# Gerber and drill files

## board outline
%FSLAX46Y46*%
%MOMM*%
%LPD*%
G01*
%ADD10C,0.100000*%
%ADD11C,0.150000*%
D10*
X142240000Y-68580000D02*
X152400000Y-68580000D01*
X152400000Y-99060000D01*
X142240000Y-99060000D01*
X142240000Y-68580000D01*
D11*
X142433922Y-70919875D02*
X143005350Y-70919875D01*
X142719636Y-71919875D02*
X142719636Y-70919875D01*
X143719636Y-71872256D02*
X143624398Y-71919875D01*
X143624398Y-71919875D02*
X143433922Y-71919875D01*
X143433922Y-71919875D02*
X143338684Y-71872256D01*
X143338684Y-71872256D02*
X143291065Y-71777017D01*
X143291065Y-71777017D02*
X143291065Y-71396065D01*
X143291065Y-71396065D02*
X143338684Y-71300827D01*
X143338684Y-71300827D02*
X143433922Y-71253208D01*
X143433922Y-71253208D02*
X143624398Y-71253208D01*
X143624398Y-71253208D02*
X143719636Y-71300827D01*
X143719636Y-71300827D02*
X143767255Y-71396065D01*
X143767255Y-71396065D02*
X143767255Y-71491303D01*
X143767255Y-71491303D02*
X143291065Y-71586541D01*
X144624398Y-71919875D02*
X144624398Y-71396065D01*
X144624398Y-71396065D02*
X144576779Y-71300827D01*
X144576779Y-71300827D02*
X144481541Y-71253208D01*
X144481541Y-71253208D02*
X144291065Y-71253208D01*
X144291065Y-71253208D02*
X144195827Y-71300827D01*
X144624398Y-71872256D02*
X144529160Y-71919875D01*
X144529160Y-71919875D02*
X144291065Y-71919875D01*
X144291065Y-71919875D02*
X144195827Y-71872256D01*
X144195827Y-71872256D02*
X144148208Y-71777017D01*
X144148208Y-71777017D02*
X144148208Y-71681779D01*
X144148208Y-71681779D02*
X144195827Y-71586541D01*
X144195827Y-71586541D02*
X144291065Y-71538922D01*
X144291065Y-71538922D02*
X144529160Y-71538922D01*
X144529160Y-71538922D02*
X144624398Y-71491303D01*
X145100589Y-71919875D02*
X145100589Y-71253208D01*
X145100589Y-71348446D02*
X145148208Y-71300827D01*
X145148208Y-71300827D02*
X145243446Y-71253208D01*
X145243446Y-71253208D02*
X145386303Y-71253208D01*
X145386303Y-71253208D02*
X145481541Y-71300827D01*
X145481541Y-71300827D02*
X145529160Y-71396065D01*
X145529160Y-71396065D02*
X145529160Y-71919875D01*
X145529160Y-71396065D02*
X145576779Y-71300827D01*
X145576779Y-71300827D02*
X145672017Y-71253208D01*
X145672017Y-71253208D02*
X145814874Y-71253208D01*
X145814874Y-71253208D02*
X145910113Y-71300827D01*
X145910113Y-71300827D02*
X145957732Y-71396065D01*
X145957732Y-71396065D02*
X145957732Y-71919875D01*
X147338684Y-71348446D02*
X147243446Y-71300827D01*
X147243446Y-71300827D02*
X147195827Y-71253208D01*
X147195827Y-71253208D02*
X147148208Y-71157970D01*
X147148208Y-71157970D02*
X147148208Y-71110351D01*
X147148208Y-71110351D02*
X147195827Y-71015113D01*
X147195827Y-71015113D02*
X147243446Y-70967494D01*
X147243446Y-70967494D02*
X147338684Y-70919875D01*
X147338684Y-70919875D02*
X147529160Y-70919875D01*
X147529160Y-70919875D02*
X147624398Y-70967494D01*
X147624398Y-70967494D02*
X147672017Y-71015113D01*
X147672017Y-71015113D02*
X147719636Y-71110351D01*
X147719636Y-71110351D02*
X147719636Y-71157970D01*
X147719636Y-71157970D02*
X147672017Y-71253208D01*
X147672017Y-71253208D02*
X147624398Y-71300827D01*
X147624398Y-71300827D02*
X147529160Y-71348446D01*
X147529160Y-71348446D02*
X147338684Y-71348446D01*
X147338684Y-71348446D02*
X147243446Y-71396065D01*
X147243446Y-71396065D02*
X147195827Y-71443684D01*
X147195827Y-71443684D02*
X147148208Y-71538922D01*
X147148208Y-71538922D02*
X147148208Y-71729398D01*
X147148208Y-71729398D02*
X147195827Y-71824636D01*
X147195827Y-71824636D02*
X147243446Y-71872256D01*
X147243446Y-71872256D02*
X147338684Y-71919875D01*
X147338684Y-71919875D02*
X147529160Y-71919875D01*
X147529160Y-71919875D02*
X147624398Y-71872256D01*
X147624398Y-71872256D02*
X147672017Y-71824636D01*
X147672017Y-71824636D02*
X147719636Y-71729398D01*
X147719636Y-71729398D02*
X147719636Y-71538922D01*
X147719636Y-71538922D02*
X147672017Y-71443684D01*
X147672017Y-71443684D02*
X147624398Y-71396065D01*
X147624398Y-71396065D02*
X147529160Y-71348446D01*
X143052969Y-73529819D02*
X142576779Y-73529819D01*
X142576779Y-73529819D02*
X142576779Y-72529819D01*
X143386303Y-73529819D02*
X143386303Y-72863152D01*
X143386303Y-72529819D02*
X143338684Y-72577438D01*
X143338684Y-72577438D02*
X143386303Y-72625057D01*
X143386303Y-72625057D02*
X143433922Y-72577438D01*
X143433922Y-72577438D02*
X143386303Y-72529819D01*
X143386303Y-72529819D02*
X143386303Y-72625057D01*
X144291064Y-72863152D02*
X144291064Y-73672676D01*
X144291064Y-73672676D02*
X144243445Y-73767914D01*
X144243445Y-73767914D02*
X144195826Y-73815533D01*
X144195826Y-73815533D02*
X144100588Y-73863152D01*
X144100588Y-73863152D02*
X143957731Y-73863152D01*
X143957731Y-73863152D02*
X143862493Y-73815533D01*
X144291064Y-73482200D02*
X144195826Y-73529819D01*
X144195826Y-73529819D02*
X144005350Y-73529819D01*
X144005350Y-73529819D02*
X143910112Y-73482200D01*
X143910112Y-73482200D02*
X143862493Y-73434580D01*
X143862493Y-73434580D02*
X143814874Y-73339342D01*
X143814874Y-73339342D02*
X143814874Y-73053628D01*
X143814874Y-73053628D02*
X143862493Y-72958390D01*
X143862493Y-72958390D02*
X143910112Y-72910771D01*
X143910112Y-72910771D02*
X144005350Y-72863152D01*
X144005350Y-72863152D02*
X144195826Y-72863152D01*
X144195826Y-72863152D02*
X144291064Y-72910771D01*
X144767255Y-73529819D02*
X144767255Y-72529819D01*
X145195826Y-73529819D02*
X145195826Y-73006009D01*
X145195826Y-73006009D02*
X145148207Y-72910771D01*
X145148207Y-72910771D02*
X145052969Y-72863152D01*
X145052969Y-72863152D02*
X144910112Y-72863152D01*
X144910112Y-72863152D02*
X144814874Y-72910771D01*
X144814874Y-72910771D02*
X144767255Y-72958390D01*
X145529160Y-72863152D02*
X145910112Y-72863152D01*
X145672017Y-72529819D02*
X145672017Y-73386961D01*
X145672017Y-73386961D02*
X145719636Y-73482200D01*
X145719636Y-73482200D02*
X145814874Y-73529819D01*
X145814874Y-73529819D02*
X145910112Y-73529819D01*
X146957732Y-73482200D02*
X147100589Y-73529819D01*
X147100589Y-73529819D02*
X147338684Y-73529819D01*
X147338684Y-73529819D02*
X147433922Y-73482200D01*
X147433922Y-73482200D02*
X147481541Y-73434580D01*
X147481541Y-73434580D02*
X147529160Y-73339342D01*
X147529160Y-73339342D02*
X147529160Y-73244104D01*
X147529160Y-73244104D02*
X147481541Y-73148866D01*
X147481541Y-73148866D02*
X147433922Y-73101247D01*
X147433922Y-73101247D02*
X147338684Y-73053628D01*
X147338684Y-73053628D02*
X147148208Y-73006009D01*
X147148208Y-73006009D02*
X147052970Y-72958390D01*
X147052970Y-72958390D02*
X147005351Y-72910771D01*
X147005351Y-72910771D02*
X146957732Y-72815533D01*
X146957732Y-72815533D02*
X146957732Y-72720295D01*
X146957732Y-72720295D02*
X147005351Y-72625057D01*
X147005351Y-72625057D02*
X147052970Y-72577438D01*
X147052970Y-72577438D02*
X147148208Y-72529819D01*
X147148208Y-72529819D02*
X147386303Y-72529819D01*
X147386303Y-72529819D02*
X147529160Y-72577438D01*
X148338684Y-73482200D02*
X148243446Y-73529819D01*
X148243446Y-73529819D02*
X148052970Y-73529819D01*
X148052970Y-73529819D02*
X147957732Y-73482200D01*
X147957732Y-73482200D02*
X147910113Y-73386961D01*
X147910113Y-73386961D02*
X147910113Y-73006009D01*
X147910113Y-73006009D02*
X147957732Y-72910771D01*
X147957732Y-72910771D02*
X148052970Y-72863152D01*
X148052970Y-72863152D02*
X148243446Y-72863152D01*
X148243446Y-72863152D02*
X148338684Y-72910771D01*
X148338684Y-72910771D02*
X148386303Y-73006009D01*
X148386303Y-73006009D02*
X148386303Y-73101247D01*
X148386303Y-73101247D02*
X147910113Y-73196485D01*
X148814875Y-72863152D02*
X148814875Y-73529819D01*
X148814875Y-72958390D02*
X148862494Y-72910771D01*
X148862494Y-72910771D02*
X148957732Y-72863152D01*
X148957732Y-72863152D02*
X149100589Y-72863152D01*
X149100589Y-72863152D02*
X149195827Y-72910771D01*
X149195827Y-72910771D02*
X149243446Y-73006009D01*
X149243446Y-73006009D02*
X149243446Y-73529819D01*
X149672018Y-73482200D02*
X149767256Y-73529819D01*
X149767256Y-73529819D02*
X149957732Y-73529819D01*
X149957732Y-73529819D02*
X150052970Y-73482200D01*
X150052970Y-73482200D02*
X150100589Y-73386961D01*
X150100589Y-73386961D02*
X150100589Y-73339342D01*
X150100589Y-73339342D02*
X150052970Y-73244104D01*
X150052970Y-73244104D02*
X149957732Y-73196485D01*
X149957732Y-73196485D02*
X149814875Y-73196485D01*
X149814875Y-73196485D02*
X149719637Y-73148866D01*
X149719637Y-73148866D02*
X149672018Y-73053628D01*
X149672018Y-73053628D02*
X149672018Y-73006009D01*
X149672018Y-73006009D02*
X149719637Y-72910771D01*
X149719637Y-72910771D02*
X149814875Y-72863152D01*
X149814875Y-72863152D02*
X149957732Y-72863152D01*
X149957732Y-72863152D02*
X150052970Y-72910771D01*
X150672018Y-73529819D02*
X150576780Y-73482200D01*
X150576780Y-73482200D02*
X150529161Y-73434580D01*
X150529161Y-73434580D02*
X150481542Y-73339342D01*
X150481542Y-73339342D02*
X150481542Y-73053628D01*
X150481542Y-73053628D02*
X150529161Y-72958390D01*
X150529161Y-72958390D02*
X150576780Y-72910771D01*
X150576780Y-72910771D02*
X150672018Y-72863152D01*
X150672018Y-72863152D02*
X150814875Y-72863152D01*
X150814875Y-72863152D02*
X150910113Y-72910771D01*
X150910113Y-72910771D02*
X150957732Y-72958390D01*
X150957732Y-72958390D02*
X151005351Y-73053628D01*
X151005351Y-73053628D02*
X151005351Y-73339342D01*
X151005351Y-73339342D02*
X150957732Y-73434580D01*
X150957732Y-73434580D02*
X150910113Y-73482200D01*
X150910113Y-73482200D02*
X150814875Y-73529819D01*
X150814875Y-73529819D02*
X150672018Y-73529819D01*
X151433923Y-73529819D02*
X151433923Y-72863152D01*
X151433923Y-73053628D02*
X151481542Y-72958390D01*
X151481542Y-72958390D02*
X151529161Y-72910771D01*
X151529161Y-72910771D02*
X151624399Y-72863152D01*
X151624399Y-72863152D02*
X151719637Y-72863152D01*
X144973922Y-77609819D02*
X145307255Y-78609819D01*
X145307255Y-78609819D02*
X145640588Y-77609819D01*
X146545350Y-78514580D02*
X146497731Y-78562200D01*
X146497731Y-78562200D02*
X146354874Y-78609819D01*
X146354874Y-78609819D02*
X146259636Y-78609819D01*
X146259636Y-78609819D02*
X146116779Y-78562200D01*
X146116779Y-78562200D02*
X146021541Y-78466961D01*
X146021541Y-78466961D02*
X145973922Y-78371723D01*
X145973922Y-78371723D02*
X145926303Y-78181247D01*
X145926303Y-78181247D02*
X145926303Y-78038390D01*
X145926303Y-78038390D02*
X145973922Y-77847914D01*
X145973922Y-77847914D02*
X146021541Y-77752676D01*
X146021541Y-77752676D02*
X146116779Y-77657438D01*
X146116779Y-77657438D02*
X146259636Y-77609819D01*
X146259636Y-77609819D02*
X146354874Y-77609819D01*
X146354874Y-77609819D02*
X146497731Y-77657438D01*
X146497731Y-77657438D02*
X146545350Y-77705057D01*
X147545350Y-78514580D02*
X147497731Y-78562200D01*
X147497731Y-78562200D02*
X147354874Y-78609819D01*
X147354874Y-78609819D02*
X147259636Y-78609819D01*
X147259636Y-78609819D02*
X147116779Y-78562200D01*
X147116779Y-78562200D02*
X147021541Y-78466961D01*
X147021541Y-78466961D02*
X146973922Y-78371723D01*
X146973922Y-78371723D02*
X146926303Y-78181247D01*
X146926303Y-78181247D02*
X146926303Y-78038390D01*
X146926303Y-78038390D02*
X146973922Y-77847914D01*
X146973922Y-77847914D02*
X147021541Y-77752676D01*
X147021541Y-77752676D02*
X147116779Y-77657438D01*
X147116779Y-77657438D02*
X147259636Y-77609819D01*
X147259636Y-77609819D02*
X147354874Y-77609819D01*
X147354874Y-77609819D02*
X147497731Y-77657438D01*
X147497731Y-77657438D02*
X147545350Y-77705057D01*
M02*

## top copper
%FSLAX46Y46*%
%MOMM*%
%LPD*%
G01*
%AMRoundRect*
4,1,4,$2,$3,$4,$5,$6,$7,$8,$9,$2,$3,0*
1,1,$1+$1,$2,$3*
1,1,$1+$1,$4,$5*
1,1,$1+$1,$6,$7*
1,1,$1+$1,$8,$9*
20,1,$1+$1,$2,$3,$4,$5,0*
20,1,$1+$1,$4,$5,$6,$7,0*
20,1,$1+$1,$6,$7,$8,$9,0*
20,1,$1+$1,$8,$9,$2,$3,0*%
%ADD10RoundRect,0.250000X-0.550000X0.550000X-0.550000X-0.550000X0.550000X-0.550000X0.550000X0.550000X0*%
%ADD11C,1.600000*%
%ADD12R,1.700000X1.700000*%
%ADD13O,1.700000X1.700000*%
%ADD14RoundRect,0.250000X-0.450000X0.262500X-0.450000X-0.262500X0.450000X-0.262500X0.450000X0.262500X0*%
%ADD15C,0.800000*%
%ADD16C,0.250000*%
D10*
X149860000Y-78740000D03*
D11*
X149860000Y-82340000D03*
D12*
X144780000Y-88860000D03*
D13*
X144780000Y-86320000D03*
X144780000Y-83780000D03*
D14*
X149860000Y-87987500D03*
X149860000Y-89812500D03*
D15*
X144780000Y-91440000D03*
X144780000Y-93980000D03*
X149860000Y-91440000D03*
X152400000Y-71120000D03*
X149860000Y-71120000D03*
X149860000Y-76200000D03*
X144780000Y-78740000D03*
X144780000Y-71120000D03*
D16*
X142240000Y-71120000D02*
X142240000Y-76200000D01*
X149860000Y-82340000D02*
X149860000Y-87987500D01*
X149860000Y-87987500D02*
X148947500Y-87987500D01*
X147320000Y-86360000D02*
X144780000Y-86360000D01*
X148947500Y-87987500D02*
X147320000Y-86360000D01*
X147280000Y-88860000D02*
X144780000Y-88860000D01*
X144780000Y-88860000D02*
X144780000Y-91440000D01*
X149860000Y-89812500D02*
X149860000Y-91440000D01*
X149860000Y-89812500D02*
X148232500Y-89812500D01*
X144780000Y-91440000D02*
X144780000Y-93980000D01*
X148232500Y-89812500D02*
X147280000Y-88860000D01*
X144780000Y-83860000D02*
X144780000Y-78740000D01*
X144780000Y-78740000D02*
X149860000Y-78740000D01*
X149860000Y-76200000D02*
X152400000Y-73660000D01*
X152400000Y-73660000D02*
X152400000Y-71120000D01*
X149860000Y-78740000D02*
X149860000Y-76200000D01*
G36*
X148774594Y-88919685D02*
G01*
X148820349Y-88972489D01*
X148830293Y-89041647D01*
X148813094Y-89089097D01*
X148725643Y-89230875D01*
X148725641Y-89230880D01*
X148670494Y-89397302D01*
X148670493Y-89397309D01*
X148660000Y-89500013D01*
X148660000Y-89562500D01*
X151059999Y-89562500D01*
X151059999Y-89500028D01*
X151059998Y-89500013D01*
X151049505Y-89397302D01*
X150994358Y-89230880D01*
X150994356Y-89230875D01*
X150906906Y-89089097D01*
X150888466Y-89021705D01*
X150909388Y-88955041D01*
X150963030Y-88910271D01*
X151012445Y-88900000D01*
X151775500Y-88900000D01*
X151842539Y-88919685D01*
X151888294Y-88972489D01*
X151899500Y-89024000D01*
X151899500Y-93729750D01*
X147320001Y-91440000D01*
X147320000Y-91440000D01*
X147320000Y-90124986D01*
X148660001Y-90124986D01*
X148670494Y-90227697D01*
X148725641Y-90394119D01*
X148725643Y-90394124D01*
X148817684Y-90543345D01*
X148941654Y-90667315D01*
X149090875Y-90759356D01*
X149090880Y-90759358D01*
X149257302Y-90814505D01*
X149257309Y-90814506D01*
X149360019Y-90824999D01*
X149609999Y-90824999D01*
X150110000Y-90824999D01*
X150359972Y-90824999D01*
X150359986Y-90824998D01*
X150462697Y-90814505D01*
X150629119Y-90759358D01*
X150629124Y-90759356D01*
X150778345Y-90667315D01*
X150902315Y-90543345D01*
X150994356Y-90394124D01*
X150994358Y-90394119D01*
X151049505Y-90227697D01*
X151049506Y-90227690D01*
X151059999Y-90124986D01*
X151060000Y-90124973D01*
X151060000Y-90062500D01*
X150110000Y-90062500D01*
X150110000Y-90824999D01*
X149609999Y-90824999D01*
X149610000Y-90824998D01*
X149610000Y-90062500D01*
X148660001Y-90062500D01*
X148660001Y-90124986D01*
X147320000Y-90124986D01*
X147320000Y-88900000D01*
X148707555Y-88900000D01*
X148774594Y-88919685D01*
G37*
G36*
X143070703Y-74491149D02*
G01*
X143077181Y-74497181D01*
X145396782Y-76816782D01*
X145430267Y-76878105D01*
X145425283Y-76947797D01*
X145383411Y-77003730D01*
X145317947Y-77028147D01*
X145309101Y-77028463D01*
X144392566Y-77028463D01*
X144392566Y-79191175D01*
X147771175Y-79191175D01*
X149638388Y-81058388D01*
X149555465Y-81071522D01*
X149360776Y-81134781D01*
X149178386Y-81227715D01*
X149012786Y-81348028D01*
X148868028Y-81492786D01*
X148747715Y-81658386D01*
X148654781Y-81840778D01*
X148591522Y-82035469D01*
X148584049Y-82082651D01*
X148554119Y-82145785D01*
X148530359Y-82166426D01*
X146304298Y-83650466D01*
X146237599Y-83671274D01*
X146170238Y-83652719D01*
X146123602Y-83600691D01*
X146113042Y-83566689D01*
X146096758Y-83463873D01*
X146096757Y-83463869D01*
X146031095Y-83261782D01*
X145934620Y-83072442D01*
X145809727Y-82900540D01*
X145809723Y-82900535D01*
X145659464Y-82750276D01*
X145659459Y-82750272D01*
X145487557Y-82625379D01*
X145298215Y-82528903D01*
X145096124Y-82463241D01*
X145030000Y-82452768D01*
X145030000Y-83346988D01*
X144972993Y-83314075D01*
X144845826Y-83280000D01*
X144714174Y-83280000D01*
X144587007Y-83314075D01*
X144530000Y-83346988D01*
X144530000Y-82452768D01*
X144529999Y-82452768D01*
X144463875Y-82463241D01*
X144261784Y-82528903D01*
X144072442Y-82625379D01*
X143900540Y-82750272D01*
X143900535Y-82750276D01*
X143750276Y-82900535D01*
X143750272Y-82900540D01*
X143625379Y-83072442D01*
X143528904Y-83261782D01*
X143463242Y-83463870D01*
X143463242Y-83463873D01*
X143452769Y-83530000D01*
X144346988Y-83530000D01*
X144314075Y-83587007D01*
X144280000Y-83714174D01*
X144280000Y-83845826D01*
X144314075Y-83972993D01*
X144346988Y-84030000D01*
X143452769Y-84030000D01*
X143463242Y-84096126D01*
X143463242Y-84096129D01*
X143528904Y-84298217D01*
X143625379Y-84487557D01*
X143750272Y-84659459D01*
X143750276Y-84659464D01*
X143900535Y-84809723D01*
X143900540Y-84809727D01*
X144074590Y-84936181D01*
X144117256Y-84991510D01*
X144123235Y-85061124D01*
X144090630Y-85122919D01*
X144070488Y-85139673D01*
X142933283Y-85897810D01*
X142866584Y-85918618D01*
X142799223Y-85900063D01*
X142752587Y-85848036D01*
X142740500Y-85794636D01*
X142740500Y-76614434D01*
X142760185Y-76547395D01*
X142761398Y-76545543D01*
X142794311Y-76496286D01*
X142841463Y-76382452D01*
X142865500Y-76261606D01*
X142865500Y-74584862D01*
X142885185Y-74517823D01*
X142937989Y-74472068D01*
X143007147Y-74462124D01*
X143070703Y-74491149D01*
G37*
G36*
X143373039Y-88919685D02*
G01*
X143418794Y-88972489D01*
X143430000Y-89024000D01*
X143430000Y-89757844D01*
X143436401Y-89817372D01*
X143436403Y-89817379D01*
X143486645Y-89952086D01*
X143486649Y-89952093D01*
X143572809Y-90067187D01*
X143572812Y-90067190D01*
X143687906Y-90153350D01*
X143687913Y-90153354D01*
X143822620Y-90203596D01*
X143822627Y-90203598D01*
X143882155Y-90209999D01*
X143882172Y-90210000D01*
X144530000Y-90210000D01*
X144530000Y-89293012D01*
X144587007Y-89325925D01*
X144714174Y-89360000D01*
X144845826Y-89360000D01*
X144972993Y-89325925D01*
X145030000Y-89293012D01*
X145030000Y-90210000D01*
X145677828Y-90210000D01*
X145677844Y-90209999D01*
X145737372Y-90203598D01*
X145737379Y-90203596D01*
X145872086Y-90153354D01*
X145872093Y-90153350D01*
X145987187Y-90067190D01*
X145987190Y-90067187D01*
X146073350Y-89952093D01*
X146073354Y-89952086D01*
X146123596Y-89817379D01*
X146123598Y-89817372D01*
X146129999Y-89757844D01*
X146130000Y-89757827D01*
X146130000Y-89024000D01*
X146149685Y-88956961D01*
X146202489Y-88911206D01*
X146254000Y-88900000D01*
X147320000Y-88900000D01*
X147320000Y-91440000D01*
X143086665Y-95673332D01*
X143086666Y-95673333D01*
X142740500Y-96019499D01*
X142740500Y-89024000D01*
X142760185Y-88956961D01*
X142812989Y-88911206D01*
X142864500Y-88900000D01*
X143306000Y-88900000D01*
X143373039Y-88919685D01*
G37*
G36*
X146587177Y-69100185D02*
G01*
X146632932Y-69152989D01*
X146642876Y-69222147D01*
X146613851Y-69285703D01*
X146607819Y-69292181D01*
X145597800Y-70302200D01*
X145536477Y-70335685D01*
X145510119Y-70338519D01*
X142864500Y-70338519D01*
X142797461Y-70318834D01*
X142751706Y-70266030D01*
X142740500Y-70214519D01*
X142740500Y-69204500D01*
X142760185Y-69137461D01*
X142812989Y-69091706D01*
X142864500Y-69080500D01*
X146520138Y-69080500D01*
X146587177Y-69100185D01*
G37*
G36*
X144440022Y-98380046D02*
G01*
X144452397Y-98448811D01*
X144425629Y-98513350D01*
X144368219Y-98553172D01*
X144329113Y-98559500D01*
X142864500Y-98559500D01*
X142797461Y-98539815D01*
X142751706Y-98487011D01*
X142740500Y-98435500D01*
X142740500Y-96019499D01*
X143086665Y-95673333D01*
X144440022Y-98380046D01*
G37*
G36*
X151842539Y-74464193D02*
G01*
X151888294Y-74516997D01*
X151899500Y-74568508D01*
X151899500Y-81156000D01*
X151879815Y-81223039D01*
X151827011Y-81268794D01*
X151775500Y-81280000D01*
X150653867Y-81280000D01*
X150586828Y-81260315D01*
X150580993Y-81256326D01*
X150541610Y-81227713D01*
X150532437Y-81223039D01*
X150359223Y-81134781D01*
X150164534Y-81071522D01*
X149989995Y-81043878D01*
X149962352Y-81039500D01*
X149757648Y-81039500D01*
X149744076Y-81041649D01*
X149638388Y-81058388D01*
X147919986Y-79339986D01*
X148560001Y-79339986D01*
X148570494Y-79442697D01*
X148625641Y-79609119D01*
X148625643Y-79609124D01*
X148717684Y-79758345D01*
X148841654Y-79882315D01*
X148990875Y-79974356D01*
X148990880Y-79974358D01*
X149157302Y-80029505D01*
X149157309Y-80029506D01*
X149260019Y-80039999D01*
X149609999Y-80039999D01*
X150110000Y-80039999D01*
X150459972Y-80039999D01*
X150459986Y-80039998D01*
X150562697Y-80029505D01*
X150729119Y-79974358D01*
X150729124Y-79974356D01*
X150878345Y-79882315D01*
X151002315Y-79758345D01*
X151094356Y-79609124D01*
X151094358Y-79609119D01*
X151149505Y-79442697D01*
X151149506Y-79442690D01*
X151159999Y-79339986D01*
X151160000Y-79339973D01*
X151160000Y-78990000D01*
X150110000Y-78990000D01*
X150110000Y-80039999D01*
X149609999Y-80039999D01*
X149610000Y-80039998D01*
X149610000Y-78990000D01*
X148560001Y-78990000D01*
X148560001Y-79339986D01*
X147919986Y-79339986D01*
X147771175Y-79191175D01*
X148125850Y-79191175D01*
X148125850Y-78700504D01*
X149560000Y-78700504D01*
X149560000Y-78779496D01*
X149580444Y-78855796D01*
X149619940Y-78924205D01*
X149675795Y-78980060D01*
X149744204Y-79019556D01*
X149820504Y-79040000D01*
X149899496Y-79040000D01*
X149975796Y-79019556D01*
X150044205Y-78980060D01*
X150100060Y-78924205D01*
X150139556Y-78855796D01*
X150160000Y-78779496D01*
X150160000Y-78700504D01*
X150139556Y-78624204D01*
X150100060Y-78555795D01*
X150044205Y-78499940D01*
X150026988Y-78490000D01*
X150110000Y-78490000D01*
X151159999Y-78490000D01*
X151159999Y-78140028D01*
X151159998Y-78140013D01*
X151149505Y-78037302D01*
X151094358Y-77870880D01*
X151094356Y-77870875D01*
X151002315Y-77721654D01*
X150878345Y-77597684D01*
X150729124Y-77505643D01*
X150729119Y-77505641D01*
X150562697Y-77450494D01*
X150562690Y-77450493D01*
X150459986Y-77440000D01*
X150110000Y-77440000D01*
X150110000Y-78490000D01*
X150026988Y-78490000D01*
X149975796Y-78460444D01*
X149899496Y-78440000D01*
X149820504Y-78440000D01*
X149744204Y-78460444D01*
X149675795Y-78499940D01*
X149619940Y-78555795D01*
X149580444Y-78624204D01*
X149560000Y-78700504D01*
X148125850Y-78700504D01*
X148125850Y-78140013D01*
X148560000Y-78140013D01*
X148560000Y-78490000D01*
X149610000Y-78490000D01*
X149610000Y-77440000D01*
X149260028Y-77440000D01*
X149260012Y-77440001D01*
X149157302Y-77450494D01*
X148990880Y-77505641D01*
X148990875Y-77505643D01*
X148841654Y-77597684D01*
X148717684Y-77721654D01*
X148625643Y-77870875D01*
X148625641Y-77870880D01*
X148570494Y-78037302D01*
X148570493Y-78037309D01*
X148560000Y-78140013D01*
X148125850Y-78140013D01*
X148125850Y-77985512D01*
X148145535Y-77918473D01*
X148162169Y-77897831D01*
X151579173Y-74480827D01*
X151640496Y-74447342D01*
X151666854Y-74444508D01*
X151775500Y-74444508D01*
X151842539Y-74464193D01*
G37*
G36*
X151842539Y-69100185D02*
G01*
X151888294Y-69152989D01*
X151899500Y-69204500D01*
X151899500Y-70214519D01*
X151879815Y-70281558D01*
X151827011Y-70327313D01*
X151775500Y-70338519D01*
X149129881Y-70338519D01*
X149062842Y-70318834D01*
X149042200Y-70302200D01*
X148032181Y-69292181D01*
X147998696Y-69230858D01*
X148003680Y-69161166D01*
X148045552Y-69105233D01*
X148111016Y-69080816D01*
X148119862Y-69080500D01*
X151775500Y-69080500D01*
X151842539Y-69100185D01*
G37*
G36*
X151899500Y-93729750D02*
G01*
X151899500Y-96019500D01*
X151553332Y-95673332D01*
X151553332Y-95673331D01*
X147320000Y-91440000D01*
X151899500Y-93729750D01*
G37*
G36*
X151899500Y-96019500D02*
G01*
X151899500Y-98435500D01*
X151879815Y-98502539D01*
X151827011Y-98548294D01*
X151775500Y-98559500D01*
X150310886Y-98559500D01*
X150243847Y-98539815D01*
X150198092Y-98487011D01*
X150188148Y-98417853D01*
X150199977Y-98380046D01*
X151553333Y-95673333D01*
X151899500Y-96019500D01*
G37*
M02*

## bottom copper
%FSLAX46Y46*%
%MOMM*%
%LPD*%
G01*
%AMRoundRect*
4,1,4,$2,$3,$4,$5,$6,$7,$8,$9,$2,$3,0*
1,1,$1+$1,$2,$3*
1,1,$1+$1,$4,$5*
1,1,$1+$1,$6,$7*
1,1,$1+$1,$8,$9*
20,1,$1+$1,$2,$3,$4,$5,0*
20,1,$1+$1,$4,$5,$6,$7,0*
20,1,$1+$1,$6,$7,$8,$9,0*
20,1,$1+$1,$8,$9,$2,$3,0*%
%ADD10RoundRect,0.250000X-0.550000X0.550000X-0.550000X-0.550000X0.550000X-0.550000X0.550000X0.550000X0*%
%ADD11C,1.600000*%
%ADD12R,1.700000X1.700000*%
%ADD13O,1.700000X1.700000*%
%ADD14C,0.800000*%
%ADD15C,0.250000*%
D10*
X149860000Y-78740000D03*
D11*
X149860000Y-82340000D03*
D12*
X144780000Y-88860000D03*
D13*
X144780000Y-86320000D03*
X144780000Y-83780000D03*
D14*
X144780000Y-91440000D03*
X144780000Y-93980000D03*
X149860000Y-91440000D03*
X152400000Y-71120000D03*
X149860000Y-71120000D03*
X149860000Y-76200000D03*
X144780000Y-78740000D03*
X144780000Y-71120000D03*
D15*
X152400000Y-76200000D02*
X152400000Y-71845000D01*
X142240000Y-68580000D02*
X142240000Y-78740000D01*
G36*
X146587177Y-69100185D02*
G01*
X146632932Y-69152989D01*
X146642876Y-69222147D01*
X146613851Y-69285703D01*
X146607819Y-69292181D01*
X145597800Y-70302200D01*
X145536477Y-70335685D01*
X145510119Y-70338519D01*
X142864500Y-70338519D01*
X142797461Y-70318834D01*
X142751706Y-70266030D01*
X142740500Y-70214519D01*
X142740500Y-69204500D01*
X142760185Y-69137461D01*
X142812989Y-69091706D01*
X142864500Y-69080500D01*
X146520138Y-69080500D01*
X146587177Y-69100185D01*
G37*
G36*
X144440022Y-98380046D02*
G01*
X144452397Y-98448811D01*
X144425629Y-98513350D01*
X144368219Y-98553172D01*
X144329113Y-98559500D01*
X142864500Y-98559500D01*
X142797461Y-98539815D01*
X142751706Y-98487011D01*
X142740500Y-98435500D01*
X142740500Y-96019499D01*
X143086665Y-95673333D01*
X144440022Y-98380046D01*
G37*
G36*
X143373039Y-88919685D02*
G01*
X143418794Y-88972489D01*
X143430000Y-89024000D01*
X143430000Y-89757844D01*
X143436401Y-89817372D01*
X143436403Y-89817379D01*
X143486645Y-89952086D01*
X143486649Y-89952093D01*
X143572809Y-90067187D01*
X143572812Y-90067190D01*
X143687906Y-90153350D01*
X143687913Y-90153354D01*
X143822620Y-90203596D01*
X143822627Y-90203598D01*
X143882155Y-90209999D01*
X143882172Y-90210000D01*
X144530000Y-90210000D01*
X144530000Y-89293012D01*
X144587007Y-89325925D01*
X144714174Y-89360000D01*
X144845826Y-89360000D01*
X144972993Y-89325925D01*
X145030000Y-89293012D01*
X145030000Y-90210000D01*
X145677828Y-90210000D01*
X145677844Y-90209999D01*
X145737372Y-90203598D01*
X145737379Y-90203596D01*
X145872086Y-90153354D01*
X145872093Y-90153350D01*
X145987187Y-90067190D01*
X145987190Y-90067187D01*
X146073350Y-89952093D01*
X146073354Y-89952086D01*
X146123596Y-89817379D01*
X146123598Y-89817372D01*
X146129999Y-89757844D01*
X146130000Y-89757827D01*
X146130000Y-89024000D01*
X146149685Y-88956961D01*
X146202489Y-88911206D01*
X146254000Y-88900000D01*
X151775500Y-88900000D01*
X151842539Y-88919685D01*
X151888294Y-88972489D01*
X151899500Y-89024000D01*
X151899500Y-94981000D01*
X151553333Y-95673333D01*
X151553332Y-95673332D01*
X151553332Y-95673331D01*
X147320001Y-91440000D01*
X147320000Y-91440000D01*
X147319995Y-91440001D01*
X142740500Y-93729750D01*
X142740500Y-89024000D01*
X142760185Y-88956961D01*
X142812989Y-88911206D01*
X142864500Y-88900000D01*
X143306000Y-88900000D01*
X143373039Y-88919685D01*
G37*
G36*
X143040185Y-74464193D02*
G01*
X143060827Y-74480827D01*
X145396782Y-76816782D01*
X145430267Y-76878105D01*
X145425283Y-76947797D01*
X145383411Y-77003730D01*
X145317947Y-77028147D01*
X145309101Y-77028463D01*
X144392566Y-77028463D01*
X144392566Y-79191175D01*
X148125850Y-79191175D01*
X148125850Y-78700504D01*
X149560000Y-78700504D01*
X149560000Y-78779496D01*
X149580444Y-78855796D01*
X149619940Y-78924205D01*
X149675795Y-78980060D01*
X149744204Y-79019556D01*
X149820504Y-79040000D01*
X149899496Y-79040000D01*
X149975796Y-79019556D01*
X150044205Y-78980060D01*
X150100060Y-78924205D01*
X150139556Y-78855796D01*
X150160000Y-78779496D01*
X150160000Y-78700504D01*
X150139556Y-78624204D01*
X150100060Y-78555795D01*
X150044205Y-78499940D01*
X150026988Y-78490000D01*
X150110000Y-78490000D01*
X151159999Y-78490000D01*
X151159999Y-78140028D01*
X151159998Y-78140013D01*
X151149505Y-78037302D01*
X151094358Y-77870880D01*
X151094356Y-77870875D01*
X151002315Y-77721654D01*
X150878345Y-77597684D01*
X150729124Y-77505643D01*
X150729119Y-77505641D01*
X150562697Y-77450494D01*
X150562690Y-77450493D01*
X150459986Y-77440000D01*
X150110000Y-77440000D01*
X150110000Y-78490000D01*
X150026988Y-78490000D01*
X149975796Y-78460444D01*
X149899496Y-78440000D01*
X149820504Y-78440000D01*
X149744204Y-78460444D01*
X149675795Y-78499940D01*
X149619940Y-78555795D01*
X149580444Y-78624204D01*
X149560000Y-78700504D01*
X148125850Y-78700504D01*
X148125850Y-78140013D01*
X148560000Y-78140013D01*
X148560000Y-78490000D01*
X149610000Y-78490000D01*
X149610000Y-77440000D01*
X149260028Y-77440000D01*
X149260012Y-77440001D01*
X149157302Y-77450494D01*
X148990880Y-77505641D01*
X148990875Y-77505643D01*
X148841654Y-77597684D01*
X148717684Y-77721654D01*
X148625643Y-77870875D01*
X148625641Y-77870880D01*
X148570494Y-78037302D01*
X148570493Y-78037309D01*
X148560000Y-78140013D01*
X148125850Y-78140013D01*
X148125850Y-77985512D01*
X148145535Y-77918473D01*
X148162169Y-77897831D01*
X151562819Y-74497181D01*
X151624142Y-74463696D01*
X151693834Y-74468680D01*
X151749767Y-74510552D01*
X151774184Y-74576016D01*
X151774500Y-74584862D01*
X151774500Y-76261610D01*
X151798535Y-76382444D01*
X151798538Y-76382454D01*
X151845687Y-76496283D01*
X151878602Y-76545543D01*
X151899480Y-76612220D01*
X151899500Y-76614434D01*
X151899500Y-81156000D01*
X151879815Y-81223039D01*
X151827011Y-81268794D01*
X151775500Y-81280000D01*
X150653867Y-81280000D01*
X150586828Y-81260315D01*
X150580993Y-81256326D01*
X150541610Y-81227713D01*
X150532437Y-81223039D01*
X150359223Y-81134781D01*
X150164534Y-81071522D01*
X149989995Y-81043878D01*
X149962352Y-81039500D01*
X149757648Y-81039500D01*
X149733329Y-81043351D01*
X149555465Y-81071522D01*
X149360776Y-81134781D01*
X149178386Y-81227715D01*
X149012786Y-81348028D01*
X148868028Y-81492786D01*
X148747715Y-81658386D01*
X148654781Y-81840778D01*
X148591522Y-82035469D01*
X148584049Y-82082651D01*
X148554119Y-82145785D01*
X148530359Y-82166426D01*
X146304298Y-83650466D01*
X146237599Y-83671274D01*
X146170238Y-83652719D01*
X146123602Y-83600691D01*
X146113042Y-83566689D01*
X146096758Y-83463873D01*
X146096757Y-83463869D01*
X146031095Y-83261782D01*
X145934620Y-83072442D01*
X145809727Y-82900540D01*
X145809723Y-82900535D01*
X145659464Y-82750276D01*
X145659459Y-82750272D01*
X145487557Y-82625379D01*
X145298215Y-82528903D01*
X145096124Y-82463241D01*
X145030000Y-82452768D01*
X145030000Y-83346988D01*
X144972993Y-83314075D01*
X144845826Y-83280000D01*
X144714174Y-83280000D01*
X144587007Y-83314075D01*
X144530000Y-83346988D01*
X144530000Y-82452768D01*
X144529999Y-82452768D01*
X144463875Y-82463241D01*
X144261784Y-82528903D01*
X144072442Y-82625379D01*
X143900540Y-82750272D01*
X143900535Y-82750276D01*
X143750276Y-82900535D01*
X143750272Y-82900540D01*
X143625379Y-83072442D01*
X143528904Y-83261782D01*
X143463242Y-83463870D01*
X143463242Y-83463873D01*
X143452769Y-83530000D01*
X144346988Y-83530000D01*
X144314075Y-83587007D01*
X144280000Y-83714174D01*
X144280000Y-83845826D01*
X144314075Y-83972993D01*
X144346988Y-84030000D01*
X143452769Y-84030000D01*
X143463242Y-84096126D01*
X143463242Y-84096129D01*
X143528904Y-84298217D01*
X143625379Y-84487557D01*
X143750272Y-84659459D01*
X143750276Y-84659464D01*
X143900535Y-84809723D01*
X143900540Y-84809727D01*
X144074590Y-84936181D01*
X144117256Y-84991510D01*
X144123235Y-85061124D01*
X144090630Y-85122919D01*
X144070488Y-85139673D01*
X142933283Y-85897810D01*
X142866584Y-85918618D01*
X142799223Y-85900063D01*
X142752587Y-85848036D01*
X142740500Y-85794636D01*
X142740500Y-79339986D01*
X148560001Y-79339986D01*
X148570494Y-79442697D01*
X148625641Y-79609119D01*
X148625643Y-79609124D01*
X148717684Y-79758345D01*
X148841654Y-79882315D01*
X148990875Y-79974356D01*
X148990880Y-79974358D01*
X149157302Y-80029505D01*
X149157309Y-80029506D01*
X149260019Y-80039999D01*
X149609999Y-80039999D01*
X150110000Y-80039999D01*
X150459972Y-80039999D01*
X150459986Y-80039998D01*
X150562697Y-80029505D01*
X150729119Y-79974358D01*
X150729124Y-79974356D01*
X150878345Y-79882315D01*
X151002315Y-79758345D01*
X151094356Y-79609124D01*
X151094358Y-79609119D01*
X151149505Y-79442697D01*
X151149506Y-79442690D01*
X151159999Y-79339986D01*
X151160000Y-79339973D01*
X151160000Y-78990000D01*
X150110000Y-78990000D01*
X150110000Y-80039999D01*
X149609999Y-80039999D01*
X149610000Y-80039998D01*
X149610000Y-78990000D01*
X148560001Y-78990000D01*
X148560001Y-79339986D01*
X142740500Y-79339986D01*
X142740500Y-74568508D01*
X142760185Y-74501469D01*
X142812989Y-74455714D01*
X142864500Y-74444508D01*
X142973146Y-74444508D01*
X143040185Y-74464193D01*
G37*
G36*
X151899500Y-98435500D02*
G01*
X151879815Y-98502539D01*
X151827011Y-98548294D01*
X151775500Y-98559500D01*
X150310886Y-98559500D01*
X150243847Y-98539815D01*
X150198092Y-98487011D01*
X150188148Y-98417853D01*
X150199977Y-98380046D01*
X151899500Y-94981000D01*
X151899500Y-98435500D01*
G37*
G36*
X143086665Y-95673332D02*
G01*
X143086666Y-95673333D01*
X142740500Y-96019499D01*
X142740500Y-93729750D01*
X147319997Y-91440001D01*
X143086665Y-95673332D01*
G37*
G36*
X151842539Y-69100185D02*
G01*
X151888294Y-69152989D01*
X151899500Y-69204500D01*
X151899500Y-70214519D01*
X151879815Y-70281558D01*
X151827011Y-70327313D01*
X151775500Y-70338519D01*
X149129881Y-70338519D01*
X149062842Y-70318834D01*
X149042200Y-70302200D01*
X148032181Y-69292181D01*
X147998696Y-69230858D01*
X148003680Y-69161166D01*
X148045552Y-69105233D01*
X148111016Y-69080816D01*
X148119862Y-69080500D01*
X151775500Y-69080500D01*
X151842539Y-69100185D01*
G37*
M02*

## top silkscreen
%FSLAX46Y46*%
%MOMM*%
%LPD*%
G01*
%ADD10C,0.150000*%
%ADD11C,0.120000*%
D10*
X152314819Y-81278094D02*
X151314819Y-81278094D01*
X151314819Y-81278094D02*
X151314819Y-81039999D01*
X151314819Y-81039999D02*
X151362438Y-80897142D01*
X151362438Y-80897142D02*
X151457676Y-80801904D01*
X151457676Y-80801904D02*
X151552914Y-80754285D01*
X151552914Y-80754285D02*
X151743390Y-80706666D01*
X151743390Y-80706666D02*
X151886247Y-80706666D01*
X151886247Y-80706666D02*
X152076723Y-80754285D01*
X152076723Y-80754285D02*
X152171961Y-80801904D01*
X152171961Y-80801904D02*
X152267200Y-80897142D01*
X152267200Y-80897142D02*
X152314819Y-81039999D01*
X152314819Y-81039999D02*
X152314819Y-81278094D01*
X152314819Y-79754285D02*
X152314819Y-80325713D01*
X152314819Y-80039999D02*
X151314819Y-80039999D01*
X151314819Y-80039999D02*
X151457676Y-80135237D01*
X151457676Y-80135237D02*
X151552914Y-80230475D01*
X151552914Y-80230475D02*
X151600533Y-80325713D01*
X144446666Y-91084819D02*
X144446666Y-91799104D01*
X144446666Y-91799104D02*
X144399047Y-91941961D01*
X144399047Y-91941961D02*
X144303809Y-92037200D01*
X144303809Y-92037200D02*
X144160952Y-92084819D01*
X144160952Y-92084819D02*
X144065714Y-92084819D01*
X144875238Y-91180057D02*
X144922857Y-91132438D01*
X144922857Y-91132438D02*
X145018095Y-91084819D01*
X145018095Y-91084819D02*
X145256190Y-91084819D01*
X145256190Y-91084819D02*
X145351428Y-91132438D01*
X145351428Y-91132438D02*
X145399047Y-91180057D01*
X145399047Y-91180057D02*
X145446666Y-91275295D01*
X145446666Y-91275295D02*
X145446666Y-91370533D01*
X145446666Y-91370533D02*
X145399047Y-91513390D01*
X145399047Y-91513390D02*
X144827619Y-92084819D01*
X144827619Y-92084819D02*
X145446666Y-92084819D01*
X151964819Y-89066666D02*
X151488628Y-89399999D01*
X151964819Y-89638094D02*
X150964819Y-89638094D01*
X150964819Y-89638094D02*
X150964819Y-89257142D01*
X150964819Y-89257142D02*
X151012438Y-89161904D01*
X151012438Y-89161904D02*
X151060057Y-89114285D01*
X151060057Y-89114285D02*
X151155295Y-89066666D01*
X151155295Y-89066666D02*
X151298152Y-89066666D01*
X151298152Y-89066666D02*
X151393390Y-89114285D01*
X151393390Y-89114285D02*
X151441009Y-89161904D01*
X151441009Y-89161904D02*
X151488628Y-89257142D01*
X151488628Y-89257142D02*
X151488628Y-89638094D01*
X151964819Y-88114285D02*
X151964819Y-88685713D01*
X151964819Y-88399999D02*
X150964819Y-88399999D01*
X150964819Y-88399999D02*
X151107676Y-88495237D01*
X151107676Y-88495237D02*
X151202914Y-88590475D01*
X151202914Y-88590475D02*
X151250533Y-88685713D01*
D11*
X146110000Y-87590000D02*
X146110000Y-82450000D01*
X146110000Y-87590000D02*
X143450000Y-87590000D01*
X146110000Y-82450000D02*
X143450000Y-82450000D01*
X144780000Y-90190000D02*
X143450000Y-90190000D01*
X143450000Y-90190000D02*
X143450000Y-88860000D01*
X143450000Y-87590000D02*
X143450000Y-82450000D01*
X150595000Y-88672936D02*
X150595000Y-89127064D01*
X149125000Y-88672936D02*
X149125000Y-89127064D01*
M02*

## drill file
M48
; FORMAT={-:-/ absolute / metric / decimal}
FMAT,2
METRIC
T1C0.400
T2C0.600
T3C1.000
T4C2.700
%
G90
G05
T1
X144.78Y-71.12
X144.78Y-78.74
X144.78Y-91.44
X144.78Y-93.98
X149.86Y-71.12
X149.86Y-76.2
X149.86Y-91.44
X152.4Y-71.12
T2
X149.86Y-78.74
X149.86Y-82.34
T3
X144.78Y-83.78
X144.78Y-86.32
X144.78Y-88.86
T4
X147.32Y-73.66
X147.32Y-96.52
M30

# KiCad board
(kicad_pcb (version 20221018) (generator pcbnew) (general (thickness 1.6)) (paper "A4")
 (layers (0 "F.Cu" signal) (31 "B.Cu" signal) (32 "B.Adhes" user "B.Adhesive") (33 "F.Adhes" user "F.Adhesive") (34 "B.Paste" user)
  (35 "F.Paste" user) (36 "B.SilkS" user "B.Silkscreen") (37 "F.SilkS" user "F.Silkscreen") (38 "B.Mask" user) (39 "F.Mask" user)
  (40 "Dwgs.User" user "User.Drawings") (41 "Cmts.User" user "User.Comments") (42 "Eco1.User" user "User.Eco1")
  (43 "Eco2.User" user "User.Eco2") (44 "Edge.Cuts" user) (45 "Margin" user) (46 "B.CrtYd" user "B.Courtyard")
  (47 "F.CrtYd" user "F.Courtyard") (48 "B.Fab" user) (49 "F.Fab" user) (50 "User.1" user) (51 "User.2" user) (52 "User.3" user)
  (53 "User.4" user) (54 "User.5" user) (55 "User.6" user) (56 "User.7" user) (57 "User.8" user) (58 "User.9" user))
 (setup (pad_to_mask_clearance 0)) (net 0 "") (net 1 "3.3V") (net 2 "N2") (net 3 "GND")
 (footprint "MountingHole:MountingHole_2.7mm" (layer "F.Cu") (at 147.32 96.52)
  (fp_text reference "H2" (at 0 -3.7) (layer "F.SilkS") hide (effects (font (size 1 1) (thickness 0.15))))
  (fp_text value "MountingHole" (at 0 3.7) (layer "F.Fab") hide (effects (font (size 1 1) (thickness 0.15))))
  (pad "" np_thru_hole circle (at 0 0) (size 2.7 2.7) (drill 2.7) (layers "*.Cu" "*.Mask")))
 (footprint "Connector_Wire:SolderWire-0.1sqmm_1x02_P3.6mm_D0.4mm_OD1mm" (layer "F.Cu") (at 149.86 78.74 -90)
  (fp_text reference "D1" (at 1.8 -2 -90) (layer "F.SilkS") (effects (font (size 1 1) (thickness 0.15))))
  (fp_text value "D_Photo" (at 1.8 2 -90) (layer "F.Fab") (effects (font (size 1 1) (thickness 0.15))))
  (pad "1" thru_hole roundrect (at 0 0 270) (size 1.6 1.6) (drill 0.6) (layers "*.Cu" "*.Mask") (roundrect_rratio 0.15625) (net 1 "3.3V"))
  (pad "2" thru_hole circle (at 3.6 0 270) (size 1.6 1.6) (drill 0.6) (layers "*.Cu" "*.Mask") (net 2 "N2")))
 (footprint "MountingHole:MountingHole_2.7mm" (layer "F.Cu") (at 147.32 73.66)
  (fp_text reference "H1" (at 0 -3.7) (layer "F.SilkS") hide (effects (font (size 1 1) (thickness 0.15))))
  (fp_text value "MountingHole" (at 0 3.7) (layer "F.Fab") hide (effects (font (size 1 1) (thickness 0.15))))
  (pad "" np_thru_hole circle (at 0 0) (size 2.7 2.7) (drill 2.7) (layers "*.Cu" "*.Mask")))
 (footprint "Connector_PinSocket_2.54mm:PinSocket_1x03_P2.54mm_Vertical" (layer "F.Cu") (at 144.78 88.86 180)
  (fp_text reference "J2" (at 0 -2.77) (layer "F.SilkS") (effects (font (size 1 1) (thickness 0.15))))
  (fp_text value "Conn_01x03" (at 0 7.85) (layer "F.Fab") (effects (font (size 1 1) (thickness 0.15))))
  (fp_line (start -1.33 1.27) (end -1.33 6.41) (stroke (width 0.12) (type solid)) (layer "F.SilkS"))
  (fp_line (start -1.33 1.27) (end 1.33 1.27) (stroke (width 0.12) (type solid)) (layer "F.SilkS"))
  (fp_line (start -1.33 6.41) (end 1.33 6.41) (stroke (width 0.12) (type solid)) (layer "F.SilkS"))
  (fp_line (start 0 -1.33) (end 1.33 -1.33) (stroke (width 0.12) (type solid)) (layer "F.SilkS"))
  (fp_line (start 1.33 -1.33) (end 1.33 0) (stroke (width 0.12) (type solid)) (layer "F.SilkS"))
  (fp_line (start 1.33 1.27) (end 1.33 6.41) (stroke (width 0.12) (type solid)) (layer "F.SilkS"))
  (pad "1" thru_hole rect (at 0 0 180) (size 1.7 1.7) (drill 1) (layers "*.Cu" "*.Mask") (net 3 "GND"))
  (pad "2" thru_hole oval (at 0 2.54 180) (size 1.7 1.7) (drill 1) (layers "*.Cu" "*.Mask") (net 2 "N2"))
  (pad "3" thru_hole oval (at 0 5.08 180) (size 1.7 1.7) (drill 1) (layers "*.Cu" "*.Mask") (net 1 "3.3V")))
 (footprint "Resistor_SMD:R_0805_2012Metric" (layer "F.Cu") (at 149.86 88.9 -90)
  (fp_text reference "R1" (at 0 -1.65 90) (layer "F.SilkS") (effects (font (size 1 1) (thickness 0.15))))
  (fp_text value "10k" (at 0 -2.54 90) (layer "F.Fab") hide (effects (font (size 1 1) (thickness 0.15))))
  (fp_line (start -0.227064 -0.735) (end 0.227064 -0.735) (stroke (width 0.12) (type solid)) (layer "F.SilkS"))
  (fp_line (start -0.227064 0.735) (end 0.227064 0.735) (stroke (width 0.12) (type solid)) (layer "F.SilkS"))
  (pad "1" smd roundrect (at -0.9125 0 270) (size 1.025 1.4) (layers "F.Cu" "F.Paste" "F.Mask") (roundrect_rratio 0.243902439) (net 2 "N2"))
  (pad "2" smd roundrect (at 0.9125 0 270) (size 1.025 1.4) (layers "F.Cu" "F.Paste" "F.Mask") (roundrect_rratio 0.243902439) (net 3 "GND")))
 (gr_rect (start 142.24 68.58) (end 152.4 99.06) (stroke (width 0.1) (type default)) (fill none) (layer "Edge.Cuts"))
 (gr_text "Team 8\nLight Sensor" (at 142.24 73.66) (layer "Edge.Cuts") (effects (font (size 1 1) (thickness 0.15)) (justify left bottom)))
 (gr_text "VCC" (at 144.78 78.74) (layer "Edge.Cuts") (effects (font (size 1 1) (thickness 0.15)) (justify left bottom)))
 (segment (start 142.24 71.12) (end 142.24 76.2) (width 0.25) (layer "F.Cu") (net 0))
 (segment (start 152.4 76.2) (end 152.4 71.845) (width 0.25) (layer "B.Cu") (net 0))
 (segment (start 149.86 82.34) (end 149.86 87.9875) (width 0.25) (layer "F.Cu") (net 2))
 (segment (start 149.86 87.9875) (end 148.9475 87.9875) (width 0.25) (layer "F.Cu") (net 2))
 (segment (start 147.32 86.36) (end 144.78 86.36) (width 0.25) (layer "F.Cu") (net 2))
 (segment (start 148.9475 87.9875) (end 147.32 86.36) (width 0.25) (layer "F.Cu") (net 2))
 (segment (start 147.28 88.86) (end 144.78 88.86) (width 0.25) (layer "F.Cu") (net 3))
 (segment (start 144.78 88.86) (end 144.78 91.44) (width 0.25) (layer "F.Cu") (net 3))
 (segment (start 149.86 89.8125) (end 149.86 91.44) (width 0.25) (layer "F.Cu") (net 3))
 (segment (start 149.86 89.8125) (end 148.2325 89.8125) (width 0.25) (layer "F.Cu") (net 3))
 (segment (start 144.78 91.44) (end 144.78 93.98) (width 0.25) (layer "F.Cu") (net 3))
 (segment (start 148.2325 89.8125) (end 147.28 88.86) (width 0.25) (layer "F.Cu") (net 3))
 (via (at 144.78 91.44) (size 0.8) (drill 0.4) (layers "F.Cu" "B.Cu") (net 3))
 (via (at 144.78 93.98) (size 0.8) (drill 0.4) (layers "F.Cu" "B.Cu") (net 3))
 (via (at 149.86 91.44) (size 0.8) (drill 0.4) (layers "F.Cu" "B.Cu") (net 3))
 (segment (start 144.78 83.86) (end 144.78 78.74) (width 0.25) (layer "F.Cu") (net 1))
 (segment (start 144.78 78.74) (end 149.86 78.74) (width 0.25) (layer "F.Cu") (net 1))
 (segment (start 149.86 76.2) (end 152.4 73.66) (width 0.25) (layer "F.Cu") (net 1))
 (segment (start 152.4 73.66) (end 152.4 71.12) (width 0.25) (layer "F.Cu") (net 1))
 (segment (start 149.86 78.74) (end 149.86 76.2) (width 0.25) (layer "F.Cu") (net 1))
 (via (at 152.4 71.12) (size 0.8) (drill 0.4) (layers "F.Cu" "B.Cu") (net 1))
 (via (at 149.86 71.12) (size 0.8) (drill 0.4) (layers "F.Cu" "B.Cu") (free) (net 1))
 (via (at 149.86 76.2) (size 0.8) (drill 0.4) (layers "F.Cu" "B.Cu") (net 1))
 (via (at 144.78 78.74) (size 0.8) (drill 0.4) (layers "F.Cu" "B.Cu") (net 1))
 (via (at 144.78 71.12) (size 0.8) (drill 0.4) (layers "F.Cu" "B.Cu") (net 1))
 (segment (start 142.24 68.58) (end 142.24 78.74) (width 0.25) (layer "B.Cu") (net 1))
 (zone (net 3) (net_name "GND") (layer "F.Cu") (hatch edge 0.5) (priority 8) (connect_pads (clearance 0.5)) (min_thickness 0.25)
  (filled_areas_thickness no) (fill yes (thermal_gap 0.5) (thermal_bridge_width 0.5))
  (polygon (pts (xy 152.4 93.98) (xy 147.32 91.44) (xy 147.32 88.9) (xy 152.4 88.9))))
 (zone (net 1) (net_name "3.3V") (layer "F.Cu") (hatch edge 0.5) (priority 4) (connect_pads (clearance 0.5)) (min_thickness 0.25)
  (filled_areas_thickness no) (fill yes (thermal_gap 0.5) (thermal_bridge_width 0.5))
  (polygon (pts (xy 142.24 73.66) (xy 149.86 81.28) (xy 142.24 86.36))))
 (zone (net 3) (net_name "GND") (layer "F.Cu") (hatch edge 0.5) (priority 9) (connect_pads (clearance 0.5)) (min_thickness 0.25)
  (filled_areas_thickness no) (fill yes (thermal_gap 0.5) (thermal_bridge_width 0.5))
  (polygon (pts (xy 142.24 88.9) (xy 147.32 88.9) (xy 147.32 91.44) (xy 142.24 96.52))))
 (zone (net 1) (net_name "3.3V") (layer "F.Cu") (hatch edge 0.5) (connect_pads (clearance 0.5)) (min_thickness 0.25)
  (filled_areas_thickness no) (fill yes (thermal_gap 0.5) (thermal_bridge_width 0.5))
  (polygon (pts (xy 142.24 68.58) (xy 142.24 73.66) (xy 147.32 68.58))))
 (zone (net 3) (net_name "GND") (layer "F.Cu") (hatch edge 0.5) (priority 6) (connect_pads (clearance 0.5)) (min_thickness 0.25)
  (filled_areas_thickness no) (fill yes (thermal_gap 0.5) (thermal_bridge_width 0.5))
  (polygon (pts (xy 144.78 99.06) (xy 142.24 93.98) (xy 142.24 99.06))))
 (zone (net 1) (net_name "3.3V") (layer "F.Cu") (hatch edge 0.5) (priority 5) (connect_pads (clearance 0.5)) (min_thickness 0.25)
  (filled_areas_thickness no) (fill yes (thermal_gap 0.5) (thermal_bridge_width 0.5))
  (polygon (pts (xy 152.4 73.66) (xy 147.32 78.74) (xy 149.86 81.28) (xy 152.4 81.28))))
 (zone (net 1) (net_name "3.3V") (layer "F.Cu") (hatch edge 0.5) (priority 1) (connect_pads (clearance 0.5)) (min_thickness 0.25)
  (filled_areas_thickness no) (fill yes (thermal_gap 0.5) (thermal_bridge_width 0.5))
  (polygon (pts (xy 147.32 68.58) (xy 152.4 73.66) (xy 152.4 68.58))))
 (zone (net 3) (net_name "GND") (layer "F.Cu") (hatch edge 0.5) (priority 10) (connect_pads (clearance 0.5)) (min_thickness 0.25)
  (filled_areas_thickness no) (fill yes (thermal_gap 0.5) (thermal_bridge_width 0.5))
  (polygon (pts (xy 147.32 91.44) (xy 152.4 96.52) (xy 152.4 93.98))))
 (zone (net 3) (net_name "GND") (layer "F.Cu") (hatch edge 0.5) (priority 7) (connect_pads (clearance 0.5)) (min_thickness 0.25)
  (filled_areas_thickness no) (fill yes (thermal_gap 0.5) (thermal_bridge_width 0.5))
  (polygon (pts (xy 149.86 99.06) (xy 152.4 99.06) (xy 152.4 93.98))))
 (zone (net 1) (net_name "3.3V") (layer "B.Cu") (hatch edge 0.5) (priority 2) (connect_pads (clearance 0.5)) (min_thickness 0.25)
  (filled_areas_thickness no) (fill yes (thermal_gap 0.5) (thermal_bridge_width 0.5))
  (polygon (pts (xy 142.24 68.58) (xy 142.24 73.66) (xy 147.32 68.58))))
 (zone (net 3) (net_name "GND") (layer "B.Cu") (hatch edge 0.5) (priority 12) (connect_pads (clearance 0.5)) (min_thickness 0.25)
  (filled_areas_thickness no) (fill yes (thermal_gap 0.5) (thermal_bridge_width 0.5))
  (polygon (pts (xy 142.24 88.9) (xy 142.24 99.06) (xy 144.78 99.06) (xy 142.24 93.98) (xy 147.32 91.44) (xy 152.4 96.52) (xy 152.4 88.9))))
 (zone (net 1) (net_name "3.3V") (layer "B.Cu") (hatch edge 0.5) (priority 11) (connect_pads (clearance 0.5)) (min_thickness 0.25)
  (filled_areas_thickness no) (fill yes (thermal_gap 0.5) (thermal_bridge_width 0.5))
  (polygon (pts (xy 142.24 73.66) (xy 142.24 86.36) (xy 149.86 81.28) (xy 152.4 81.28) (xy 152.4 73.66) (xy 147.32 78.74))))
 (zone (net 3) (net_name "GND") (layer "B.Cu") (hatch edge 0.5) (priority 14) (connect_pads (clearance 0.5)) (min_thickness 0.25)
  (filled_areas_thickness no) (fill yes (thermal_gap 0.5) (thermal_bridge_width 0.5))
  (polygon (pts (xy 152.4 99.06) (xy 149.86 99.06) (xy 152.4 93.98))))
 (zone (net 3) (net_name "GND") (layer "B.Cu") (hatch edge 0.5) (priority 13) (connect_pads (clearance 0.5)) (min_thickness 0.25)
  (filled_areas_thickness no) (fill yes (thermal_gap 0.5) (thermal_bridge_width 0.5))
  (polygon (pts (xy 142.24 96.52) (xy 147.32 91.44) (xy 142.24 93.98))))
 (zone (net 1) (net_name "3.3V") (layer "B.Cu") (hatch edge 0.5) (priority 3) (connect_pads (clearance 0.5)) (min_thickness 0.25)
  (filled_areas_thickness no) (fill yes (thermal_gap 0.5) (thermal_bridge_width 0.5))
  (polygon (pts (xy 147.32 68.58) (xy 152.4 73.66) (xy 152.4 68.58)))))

